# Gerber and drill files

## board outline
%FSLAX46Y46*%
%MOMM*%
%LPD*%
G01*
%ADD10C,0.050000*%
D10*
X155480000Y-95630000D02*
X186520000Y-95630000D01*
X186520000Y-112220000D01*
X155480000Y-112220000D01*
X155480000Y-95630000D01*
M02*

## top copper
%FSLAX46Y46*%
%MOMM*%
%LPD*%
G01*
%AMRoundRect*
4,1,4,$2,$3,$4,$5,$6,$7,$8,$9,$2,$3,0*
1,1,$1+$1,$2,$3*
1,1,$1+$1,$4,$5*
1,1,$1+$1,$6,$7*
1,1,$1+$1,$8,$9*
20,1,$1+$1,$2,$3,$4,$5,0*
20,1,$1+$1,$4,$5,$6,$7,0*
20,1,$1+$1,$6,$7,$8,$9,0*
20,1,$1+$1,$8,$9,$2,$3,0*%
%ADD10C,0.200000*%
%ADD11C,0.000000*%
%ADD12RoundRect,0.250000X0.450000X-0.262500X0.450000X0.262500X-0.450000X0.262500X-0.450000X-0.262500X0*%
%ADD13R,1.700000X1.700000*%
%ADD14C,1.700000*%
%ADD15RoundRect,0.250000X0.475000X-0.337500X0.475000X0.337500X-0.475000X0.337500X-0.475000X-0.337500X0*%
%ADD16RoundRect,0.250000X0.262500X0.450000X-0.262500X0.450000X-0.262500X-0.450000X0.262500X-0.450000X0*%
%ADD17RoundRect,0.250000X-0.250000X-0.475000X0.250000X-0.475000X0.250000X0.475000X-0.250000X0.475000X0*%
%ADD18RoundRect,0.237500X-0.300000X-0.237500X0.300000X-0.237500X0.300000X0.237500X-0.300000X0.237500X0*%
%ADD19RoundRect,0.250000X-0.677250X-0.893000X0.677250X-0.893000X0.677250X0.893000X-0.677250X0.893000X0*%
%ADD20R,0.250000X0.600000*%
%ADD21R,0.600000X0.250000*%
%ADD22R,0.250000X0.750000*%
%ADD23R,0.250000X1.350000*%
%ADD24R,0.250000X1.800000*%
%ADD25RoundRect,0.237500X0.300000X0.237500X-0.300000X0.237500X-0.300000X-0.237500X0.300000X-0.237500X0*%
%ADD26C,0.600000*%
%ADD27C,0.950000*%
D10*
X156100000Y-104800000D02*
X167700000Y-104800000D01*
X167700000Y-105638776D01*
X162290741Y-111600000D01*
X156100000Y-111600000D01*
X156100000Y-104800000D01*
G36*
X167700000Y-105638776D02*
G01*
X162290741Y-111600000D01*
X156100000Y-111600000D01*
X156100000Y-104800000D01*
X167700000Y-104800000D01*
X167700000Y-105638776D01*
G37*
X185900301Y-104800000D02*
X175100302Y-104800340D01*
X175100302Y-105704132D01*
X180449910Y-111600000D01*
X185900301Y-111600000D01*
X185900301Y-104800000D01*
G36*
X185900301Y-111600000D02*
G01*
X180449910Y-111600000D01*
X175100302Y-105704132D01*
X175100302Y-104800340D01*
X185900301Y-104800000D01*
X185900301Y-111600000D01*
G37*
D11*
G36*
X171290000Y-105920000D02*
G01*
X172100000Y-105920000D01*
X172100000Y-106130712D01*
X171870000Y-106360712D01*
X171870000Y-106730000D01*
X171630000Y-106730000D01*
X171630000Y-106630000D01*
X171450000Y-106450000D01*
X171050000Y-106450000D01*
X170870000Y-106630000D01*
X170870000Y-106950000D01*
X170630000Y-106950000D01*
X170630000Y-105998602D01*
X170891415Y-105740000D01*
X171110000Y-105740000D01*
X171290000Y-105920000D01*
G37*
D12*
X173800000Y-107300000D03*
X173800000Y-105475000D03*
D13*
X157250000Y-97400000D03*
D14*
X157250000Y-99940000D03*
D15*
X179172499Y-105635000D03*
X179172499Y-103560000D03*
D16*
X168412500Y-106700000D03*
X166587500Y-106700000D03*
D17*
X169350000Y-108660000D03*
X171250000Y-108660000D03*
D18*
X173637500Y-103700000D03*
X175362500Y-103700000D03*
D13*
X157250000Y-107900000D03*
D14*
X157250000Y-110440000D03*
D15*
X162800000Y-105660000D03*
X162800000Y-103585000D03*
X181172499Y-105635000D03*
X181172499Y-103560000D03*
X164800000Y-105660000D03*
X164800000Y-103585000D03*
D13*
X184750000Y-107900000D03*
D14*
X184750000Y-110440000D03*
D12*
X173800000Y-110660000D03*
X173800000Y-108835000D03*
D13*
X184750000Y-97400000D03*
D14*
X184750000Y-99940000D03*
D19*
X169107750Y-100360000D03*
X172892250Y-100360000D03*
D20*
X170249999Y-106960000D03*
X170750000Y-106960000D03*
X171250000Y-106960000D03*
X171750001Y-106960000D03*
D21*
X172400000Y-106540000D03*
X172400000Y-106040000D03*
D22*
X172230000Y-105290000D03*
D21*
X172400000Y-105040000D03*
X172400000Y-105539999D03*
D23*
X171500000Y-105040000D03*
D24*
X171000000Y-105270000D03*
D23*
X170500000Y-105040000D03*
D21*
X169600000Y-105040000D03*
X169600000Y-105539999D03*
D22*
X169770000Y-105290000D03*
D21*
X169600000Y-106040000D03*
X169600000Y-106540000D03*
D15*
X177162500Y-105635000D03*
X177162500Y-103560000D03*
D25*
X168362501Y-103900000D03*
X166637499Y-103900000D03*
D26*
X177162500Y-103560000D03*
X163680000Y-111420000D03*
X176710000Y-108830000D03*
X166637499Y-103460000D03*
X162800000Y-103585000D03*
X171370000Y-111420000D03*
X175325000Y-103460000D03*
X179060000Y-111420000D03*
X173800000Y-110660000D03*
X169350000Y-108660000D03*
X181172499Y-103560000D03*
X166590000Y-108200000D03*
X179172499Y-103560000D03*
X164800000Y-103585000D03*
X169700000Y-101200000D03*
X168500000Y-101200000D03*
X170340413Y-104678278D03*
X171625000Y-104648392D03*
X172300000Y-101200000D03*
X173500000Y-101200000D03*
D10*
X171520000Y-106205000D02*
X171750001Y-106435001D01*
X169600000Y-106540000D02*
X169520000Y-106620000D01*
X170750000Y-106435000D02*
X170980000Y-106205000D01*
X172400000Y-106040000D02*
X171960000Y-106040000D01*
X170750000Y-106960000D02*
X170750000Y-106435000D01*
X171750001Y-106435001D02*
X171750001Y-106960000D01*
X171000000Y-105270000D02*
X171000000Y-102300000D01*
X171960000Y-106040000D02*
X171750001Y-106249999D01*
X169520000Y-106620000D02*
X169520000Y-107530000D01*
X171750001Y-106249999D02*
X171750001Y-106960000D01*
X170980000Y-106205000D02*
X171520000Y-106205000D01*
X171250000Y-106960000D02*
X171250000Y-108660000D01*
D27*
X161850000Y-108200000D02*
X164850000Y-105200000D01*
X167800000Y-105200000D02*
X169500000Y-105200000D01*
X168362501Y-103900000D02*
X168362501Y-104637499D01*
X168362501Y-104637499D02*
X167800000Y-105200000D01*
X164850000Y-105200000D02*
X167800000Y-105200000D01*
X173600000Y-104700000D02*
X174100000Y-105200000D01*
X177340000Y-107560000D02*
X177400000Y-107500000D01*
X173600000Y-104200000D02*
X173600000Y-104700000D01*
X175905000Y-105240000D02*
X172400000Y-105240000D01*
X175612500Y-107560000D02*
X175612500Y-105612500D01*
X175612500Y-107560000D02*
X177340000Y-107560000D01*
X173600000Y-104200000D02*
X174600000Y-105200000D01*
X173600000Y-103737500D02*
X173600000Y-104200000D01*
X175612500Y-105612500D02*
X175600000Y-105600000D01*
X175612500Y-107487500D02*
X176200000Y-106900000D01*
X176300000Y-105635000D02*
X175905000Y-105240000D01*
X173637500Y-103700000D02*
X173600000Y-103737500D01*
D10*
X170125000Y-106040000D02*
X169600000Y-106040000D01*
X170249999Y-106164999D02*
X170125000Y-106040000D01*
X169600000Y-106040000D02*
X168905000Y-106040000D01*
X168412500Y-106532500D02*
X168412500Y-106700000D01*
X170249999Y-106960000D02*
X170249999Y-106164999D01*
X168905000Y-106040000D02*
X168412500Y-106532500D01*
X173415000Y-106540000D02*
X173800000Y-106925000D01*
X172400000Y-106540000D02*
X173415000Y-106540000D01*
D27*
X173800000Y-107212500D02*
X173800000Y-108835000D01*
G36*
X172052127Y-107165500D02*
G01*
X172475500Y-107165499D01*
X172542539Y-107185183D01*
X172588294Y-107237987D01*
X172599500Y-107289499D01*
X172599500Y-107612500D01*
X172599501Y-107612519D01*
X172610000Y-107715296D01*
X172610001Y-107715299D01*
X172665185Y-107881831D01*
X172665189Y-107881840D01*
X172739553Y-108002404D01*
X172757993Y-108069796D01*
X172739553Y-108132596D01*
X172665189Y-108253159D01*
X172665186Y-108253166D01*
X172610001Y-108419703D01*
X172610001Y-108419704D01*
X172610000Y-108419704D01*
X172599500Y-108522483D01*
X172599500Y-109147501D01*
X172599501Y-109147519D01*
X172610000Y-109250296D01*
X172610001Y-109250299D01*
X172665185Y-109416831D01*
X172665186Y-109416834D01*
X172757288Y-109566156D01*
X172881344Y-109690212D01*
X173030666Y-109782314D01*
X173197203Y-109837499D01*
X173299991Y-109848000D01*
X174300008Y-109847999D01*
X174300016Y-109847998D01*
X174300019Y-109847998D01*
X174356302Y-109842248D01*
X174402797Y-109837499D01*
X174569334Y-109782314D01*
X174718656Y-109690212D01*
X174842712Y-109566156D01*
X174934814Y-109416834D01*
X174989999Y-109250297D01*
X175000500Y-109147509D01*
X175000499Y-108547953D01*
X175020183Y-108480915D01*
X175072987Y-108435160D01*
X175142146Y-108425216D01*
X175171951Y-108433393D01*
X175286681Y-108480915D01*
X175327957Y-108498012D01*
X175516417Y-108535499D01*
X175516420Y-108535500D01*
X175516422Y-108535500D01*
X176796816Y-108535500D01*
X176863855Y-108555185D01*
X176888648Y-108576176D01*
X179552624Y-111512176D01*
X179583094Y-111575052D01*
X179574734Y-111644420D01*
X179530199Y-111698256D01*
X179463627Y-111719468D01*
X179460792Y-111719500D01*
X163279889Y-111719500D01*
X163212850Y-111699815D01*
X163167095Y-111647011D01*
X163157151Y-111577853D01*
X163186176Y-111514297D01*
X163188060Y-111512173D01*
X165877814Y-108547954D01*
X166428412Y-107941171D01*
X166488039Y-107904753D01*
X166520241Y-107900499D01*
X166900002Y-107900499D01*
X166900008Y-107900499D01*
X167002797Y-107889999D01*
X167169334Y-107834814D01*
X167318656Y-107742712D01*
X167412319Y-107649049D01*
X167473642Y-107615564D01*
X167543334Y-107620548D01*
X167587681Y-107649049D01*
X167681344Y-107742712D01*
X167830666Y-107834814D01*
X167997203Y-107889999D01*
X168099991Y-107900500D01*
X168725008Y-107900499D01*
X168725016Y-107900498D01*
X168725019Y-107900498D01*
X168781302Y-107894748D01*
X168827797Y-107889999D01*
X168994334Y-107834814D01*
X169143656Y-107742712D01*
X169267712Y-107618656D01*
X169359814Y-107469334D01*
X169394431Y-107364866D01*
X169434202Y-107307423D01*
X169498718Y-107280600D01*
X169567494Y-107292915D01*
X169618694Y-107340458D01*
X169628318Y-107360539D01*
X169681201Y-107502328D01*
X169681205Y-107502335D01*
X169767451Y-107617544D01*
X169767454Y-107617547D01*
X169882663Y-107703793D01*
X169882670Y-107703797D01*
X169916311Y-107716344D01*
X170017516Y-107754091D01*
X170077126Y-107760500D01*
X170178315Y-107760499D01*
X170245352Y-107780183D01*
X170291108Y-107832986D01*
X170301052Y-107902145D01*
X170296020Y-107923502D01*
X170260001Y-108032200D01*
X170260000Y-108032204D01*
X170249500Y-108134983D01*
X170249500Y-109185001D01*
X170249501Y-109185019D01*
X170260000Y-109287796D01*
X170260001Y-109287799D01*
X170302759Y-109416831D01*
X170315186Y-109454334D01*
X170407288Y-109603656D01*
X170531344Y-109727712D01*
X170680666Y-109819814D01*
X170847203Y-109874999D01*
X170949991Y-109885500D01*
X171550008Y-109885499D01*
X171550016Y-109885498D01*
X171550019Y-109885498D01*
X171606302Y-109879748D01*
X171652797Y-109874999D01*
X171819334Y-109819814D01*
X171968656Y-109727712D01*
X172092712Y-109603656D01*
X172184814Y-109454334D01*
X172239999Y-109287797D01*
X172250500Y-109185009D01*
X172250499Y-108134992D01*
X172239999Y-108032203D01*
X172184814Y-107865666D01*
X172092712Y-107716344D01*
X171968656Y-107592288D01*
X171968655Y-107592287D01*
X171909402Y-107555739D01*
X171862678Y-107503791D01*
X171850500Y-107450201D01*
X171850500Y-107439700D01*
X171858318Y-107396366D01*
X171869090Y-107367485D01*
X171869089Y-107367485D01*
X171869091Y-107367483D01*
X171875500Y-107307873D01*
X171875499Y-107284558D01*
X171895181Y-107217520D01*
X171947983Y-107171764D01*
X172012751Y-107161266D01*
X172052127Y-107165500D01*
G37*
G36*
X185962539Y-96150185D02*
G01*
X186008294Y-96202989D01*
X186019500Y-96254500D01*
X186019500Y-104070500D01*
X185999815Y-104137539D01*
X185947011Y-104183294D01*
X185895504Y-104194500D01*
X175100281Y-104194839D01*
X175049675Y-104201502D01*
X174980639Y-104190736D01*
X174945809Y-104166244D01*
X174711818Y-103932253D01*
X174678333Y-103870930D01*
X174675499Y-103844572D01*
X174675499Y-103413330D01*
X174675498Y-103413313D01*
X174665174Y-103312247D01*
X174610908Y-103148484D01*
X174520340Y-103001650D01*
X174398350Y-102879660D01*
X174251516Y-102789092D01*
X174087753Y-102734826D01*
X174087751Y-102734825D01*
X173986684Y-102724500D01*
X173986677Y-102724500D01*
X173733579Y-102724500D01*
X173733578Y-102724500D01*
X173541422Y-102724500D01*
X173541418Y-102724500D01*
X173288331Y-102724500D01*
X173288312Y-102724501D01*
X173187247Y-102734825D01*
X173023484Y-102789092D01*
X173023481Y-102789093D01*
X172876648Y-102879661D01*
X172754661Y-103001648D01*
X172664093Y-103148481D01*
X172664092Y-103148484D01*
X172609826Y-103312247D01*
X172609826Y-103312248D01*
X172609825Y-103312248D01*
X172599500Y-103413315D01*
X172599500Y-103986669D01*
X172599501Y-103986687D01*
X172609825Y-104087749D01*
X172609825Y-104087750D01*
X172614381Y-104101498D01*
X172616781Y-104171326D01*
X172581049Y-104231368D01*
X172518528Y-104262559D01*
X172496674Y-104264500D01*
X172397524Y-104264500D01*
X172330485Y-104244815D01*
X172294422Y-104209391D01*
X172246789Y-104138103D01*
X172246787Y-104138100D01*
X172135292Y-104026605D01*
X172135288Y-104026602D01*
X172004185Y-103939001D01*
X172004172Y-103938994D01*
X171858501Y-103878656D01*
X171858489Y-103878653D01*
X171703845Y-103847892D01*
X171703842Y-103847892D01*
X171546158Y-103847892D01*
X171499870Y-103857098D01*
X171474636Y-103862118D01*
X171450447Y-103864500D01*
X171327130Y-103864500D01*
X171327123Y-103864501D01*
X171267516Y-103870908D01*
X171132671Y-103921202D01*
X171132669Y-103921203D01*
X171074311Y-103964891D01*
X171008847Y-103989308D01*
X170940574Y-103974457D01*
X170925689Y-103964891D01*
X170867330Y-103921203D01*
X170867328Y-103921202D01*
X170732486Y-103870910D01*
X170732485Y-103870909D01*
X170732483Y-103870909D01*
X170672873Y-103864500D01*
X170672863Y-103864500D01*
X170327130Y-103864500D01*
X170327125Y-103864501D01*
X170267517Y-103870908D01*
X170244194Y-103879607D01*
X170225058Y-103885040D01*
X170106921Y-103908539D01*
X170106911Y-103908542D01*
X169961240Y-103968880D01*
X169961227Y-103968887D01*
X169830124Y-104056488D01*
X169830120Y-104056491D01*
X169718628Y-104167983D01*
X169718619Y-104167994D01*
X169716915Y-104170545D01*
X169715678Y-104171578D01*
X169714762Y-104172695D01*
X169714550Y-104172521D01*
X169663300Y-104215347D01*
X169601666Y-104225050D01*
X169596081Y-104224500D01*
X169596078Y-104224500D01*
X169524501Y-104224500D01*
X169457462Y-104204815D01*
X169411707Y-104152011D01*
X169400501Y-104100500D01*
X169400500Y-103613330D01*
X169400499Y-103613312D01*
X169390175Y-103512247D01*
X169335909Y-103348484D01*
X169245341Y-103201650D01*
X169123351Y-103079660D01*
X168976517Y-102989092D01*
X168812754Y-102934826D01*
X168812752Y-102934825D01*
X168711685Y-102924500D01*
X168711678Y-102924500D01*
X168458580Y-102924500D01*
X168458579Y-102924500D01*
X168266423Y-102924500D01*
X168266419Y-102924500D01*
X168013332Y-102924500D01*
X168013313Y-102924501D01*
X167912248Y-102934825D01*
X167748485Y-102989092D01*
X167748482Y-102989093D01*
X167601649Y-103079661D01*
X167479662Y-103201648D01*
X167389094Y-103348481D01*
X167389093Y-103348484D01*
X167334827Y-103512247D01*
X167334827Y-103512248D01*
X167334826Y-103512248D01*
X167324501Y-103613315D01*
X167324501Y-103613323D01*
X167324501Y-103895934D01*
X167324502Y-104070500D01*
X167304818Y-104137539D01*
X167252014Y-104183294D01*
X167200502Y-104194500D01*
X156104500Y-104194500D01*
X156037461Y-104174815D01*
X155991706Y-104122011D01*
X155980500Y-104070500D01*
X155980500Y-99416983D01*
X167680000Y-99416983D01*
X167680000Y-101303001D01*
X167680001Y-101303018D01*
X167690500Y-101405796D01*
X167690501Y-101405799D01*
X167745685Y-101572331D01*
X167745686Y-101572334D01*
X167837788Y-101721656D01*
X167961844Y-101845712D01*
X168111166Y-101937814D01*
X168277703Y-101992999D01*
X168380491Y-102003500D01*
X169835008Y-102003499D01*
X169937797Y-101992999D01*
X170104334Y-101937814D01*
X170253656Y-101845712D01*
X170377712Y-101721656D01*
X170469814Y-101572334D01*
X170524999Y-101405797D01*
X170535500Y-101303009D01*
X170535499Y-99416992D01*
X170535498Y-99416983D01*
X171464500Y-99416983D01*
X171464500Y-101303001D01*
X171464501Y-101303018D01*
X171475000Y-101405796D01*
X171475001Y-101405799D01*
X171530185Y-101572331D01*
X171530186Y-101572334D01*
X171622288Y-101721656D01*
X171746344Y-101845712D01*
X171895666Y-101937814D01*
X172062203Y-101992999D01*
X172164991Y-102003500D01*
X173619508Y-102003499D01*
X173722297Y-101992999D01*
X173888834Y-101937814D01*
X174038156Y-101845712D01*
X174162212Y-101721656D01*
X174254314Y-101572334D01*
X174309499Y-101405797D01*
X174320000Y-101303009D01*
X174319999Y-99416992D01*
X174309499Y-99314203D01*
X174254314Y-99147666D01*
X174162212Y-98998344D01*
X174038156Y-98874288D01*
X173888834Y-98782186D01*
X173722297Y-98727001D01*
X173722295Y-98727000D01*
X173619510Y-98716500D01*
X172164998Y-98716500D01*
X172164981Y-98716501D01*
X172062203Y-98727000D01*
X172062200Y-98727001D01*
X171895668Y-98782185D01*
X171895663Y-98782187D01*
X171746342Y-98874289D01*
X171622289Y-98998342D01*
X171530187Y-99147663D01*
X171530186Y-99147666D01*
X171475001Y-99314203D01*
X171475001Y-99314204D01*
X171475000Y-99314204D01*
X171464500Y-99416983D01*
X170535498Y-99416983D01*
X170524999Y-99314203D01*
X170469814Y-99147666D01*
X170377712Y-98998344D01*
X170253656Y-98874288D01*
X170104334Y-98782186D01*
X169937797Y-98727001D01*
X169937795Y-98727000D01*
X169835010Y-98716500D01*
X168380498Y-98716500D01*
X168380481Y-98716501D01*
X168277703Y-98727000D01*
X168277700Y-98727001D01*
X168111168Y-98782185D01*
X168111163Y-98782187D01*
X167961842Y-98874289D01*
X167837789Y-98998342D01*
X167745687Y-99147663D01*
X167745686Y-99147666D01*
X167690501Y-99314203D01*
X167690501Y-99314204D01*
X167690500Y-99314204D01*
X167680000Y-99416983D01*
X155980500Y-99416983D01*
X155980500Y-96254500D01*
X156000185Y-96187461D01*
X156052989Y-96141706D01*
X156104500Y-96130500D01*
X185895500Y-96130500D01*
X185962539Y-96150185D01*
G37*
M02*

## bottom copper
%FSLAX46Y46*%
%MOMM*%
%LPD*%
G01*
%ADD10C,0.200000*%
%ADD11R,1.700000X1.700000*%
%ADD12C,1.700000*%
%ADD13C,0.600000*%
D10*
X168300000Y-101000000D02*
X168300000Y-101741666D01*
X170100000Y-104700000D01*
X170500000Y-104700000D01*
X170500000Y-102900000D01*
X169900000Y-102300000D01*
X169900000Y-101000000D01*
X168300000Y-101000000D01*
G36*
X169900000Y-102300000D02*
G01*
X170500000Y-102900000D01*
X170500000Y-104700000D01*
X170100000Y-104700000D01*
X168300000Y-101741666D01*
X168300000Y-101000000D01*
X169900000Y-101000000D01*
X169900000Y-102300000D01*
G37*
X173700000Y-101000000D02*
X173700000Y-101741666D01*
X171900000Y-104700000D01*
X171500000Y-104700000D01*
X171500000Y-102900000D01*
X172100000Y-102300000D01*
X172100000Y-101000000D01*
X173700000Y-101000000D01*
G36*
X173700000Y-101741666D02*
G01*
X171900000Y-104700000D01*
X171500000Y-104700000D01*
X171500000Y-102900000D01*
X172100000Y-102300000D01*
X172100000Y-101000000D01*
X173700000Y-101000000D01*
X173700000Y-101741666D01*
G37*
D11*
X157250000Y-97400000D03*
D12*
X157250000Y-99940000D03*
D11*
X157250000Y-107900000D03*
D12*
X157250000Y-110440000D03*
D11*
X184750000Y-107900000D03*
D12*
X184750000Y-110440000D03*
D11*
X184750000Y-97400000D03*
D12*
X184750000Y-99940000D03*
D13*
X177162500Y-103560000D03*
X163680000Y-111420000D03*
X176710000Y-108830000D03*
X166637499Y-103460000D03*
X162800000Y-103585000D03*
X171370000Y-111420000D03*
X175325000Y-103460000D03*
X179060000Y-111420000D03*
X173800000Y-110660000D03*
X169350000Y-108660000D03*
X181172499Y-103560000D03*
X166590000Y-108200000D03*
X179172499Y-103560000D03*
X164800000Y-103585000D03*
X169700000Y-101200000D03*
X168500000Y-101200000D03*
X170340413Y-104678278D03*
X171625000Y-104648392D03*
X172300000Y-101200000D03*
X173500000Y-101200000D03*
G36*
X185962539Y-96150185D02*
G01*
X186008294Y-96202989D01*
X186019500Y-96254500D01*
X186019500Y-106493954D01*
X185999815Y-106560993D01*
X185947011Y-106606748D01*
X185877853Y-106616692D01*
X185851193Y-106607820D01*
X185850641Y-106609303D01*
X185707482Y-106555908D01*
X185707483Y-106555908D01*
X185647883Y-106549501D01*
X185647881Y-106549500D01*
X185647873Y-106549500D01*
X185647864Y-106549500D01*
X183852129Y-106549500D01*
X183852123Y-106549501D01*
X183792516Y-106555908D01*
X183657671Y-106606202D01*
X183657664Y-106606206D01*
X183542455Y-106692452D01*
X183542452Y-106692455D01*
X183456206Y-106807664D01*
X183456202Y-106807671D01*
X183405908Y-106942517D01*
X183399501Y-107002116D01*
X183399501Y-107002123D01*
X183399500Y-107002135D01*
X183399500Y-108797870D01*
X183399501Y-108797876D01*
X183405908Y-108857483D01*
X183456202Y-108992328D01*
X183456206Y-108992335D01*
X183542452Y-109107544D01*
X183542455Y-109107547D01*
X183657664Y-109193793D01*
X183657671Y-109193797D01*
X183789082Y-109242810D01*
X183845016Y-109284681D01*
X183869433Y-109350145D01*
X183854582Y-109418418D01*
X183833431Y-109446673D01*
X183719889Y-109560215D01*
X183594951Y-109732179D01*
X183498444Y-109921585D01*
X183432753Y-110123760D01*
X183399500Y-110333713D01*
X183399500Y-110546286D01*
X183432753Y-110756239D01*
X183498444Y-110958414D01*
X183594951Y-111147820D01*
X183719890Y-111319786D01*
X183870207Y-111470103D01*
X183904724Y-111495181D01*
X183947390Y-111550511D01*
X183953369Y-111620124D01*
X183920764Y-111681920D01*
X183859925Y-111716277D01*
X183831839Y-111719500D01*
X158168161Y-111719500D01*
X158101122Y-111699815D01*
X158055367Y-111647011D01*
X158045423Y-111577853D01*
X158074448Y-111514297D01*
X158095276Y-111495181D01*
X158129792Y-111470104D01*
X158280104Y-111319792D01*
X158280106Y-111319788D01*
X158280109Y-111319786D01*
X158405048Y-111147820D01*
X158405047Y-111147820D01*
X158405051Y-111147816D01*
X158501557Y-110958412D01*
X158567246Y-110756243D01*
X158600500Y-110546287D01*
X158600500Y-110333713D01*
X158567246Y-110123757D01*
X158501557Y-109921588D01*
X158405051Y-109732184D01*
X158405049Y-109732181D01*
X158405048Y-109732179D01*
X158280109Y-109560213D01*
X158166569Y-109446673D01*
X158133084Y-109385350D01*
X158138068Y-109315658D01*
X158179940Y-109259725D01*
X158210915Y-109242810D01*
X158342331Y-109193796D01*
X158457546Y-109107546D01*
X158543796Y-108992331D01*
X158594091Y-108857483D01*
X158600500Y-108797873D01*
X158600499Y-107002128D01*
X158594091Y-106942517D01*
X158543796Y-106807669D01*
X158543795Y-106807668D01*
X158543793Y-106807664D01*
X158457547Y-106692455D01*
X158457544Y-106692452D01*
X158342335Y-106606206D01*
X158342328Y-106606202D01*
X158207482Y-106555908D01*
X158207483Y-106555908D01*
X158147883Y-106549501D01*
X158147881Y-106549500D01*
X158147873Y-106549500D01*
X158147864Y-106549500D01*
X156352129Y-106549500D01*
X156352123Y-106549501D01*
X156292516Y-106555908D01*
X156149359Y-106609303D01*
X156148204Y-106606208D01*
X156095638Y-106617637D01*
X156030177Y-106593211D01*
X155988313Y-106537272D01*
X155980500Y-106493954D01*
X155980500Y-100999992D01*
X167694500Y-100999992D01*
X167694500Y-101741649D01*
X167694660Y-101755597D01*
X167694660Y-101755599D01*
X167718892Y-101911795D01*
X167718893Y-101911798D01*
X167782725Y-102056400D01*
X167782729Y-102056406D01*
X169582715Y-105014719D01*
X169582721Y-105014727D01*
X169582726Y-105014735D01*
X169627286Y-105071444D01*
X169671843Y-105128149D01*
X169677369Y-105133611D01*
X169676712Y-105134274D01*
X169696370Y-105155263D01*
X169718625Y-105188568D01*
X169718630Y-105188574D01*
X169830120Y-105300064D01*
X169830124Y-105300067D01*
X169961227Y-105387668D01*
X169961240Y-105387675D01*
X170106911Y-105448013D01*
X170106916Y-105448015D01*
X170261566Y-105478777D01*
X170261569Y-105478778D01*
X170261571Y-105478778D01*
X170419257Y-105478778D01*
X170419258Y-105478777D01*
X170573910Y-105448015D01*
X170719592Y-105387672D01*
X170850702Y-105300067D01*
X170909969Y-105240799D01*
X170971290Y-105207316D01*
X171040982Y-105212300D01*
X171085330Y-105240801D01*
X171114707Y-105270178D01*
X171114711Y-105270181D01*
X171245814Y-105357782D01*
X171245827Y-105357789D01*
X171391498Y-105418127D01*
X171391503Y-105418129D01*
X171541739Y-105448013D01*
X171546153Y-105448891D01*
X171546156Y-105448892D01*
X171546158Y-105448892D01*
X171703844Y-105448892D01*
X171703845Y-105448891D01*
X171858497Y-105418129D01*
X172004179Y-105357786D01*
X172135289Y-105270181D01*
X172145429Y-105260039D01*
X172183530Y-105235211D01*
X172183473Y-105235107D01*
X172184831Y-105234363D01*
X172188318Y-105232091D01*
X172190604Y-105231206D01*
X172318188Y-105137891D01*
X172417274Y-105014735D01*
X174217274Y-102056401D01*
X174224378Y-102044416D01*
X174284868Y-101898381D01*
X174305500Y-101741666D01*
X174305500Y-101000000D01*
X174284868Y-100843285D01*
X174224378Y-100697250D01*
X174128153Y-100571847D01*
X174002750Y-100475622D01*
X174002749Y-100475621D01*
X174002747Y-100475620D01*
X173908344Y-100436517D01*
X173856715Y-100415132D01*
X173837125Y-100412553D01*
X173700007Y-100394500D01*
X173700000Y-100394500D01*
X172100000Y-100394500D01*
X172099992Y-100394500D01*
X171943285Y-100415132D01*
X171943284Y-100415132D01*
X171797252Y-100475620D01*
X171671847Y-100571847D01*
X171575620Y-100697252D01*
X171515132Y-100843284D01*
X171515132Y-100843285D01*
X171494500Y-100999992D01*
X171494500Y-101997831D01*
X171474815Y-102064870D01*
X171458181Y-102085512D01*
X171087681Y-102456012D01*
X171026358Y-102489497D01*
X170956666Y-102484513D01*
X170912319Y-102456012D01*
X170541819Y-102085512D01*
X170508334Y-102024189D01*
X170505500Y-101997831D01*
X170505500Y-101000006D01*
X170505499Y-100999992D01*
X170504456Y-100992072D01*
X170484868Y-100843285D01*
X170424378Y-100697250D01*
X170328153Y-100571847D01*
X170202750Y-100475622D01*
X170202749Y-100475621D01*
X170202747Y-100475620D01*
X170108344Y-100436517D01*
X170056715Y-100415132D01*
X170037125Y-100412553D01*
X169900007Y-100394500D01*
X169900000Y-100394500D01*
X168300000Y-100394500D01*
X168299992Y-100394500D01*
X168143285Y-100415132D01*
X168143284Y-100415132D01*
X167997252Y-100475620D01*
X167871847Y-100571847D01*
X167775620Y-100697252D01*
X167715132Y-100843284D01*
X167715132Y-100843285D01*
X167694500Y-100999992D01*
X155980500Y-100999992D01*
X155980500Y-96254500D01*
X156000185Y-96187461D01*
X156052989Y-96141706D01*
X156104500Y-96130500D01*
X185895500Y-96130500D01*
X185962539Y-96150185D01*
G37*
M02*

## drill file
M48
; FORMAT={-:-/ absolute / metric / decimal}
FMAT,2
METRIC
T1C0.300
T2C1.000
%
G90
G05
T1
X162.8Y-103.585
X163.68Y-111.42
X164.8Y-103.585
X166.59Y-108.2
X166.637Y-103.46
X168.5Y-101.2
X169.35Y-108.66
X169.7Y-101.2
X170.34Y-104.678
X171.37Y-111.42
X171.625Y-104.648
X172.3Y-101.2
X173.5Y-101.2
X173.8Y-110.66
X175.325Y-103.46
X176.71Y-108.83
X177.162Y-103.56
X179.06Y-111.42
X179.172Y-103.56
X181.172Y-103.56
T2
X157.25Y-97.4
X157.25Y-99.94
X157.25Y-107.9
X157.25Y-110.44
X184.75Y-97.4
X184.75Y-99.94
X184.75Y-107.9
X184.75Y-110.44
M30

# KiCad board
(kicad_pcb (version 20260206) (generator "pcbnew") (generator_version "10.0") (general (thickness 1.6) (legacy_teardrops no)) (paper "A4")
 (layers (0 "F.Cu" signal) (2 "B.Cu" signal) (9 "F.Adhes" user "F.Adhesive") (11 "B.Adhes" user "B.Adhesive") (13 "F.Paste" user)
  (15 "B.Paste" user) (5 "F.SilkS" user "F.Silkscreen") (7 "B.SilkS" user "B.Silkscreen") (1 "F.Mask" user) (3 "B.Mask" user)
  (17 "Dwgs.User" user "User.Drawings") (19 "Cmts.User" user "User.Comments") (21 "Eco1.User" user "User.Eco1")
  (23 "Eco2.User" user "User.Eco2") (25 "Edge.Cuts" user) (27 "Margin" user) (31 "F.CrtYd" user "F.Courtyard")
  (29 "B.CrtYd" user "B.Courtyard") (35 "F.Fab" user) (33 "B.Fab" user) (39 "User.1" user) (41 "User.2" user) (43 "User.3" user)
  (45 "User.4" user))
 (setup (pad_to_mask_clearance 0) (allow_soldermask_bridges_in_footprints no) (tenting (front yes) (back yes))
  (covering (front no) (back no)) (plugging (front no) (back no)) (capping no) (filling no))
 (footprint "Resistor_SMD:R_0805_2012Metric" (layer "F.Cu") (at 173.8 106.3875 90)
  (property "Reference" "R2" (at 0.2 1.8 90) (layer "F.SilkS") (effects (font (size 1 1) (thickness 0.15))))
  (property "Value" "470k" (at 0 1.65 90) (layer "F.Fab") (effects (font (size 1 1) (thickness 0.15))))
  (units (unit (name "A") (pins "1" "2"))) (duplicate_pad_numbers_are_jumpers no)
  (pad "1" smd roundrect (at -0.9125 0 90) (size 1.025 1.4) (layers "F.Cu" "F.Mask" "F.Paste") (roundrect_rratio 0.243902)
   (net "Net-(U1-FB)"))
  (pad "2" smd roundrect (at 0.9125 0 90) (size 1.025 1.4) (layers "F.Cu" "F.Mask" "F.Paste") (roundrect_rratio 0.243902) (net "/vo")))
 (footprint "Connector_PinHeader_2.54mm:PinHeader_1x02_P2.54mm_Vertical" (layer "F.Cu") (at 157.25 97.4)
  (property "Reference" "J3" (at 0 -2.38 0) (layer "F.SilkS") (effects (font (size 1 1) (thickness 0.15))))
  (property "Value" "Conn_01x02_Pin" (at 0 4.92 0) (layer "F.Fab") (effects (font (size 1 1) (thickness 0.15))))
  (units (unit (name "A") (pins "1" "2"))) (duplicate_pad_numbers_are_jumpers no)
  (pad "1" thru_hole rect (at 0 0) (size 1.7 1.7) (drill 1) (layers "*.Cu" "*.Mask") (remove_unused_layers no) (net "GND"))
  (pad "2" thru_hole circle (at 0 2.54) (size 1.7 1.7) (drill 1) (layers "*.Cu" "*.Mask") (remove_unused_layers no) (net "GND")))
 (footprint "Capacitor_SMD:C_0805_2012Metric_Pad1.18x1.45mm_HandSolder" (layer "F.Cu") (at 179.172499 104.5975 90)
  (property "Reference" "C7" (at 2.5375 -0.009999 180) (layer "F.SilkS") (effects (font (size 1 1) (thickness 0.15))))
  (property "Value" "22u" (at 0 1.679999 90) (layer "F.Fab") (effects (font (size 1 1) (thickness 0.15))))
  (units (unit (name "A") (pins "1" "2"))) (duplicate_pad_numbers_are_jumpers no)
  (pad "1" smd roundrect (at -1.0375 0 90) (size 1.175 1.45) (layers "F.Cu" "F.Mask" "F.Paste") (roundrect_rratio 0.212766) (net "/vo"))
  (pad "2" smd roundrect (at 1.0375 0 90) (size 1.175 1.45) (layers "F.Cu" "F.Mask" "F.Paste") (roundrect_rratio 0.212766) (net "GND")))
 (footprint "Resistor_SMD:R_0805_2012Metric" (layer "F.Cu") (at 167.5 106.7 180)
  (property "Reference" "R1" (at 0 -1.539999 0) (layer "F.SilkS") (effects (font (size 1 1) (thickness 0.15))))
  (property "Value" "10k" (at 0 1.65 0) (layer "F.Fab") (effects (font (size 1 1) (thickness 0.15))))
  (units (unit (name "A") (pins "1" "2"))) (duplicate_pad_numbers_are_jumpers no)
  (pad "1" smd roundrect (at -0.9125 0 180) (size 1.025 1.4) (layers "F.Cu" "F.Mask" "F.Paste") (roundrect_rratio 0.243902)
   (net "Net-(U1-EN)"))
  (pad "2" smd roundrect (at 0.9125 0 180) (size 1.025 1.4) (layers "F.Cu" "F.Mask" "F.Paste") (roundrect_rratio 0.243902) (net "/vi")))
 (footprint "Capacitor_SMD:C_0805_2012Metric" (layer "F.Cu") (at 170.3 108.66)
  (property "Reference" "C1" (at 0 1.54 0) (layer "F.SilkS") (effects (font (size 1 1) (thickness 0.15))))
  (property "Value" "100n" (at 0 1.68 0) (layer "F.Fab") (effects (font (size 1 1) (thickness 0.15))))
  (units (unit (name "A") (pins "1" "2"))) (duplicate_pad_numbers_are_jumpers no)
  (pad "1" smd roundrect (at -0.95 0) (size 1 1.45) (layers "F.Cu" "F.Mask" "F.Paste") (roundrect_rratio 0.25) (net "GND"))
  (pad "2" smd roundrect (at 0.95 0) (size 1 1.45) (layers "F.Cu" "F.Mask" "F.Paste") (roundrect_rratio 0.25) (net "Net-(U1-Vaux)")))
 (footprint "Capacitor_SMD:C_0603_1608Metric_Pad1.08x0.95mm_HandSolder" (layer "F.Cu") (at 174.5 103.7)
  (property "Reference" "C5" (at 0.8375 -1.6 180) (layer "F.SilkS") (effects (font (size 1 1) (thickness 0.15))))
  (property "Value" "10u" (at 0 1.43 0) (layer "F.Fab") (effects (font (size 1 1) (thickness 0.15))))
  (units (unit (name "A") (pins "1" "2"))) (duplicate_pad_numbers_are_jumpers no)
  (pad "1" smd roundrect (at -0.8625 0) (size 1.075 0.95) (layers "F.Cu" "F.Mask" "F.Paste") (roundrect_rratio 0.25) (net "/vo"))
  (pad "2" smd roundrect (at 0.8625 0) (size 1.075 0.95) (layers "F.Cu" "F.Mask" "F.Paste") (roundrect_rratio 0.25) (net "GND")))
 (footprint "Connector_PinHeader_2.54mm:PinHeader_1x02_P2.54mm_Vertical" (layer "F.Cu") (at 157.25 107.9)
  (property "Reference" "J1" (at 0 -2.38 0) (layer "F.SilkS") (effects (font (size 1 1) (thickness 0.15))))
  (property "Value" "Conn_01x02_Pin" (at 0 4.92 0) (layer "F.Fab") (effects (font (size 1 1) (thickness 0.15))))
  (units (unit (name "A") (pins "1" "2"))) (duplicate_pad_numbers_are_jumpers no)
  (pad "1" thru_hole rect (at 0 0) (size 1.7 1.7) (drill 1) (layers "*.Cu" "*.Mask") (remove_unused_layers no) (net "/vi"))
  (pad "2" thru_hole circle (at 0 2.54) (size 1.7 1.7) (drill 1) (layers "*.Cu" "*.Mask") (remove_unused_layers no) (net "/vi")))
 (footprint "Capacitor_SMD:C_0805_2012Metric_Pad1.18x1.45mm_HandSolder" (layer "F.Cu") (at 162.8 104.6225 90)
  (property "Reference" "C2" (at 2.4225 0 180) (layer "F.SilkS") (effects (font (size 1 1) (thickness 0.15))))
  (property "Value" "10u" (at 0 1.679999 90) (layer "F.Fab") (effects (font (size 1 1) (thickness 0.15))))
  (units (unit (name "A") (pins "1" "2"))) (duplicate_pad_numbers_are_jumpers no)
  (pad "1" smd roundrect (at -1.0375 0 90) (size 1.175 1.45) (layers "F.Cu" "F.Mask" "F.Paste") (roundrect_rratio 0.212766) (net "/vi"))
  (pad "2" smd roundrect (at 1.0375 0 90) (size 1.175 1.45) (layers "F.Cu" "F.Mask" "F.Paste") (roundrect_rratio 0.212766) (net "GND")))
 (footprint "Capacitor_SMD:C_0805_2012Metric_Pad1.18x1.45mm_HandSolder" (layer "F.Cu") (at 181.172499 104.5975 90)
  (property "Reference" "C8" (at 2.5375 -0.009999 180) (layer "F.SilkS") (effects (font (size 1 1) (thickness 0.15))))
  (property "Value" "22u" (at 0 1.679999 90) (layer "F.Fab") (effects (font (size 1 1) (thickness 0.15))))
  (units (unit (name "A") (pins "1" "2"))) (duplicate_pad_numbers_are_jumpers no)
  (pad "1" smd roundrect (at -1.0375 0 90) (size 1.175 1.45) (layers "F.Cu" "F.Mask" "F.Paste") (roundrect_rratio 0.212766) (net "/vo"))
  (pad "2" smd roundrect (at 1.0375 0 90) (size 1.175 1.45) (layers "F.Cu" "F.Mask" "F.Paste") (roundrect_rratio 0.212766) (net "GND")))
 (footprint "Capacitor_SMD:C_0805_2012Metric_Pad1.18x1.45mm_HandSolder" (layer "F.Cu") (at 164.8 104.6225 90)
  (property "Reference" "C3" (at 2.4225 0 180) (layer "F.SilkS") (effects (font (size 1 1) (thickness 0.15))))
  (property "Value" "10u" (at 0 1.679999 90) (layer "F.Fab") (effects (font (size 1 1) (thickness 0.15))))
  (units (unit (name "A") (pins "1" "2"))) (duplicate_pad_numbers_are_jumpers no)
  (pad "1" smd roundrect (at -1.0375 0 90) (size 1.175 1.45) (layers "F.Cu" "F.Mask" "F.Paste") (roundrect_rratio 0.212766) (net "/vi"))
  (pad "2" smd roundrect (at 1.0375 0 90) (size 1.175 1.45) (layers "F.Cu" "F.Mask" "F.Paste") (roundrect_rratio 0.212766) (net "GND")))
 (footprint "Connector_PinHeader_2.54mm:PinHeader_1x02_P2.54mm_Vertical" (layer "F.Cu") (at 184.75 107.9)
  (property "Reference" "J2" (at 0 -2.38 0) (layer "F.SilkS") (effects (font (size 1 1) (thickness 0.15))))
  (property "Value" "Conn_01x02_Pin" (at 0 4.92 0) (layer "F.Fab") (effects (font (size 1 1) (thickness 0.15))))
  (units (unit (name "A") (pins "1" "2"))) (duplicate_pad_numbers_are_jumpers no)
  (pad "1" thru_hole rect (at 0 0) (size 1.7 1.7) (drill 1) (layers "*.Cu" "*.Mask") (remove_unused_layers no) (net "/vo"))
  (pad "2" thru_hole circle (at 0 2.54) (size 1.7 1.7) (drill 1) (layers "*.Cu" "*.Mask") (remove_unused_layers no) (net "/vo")))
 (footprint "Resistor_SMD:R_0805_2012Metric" (layer "F.Cu") (at 173.8 109.7475 90)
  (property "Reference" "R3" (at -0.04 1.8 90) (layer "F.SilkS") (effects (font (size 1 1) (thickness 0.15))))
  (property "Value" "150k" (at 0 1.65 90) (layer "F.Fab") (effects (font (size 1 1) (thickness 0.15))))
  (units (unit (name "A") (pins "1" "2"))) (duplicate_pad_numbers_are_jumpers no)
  (pad "1" smd roundrect (at -0.9125 0 90) (size 1.025 1.4) (layers "F.Cu" "F.Mask" "F.Paste") (roundrect_rratio 0.243902) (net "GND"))
  (pad "2" smd roundrect (at 0.9125 0 90) (size 1.025 1.4) (layers "F.Cu" "F.Mask" "F.Paste") (roundrect_rratio 0.243902)
   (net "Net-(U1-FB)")))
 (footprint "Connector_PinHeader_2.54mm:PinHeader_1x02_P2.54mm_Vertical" (layer "F.Cu") (at 184.75 97.4)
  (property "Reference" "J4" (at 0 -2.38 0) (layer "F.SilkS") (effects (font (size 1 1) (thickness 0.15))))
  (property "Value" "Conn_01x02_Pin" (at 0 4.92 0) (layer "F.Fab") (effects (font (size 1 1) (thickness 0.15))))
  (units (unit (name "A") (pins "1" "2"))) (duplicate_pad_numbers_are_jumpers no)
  (pad "1" thru_hole rect (at 0 0) (size 1.7 1.7) (drill 1) (layers "*.Cu" "*.Mask") (remove_unused_layers no) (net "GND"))
  (pad "2" thru_hole circle (at 0 2.54) (size 1.7 1.7) (drill 1) (layers "*.Cu" "*.Mask") (remove_unused_layers no) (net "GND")))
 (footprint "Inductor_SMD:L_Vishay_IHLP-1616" (layer "F.Cu") (at 171 100.36)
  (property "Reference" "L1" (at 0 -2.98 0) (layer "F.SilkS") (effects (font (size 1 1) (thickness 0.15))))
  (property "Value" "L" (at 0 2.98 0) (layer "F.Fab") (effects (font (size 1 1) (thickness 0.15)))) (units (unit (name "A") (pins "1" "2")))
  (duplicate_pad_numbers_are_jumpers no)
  (pad "1" smd roundrect (at -1.89225 0) (size 1.8545 2.286) (layers "F.Cu" "F.Mask" "F.Paste") (roundrect_rratio 0.134807)
   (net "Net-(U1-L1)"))
  (pad "2" smd roundrect (at 1.89225 0) (size 1.8545 2.286) (layers "F.Cu" "F.Mask" "F.Paste") (roundrect_rratio 0.134807)
   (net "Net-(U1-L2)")))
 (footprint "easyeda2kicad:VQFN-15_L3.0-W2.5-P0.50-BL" (layer "F.Cu") (at 171 106)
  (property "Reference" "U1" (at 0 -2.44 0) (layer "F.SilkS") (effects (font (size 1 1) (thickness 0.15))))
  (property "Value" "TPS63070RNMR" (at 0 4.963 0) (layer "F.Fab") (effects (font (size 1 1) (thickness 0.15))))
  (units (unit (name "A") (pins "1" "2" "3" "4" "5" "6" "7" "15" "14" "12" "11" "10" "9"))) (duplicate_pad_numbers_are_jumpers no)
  (pad "1" smd rect (at -0.750001 0.96 180) (size 0.25 0.6) (layers "F.Cu" "F.Mask" "F.Paste") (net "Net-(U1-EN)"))
  (pad "2" smd rect (at -0.25 0.96 180) (size 0.25 0.6) (layers "F.Cu" "F.Mask" "F.Paste") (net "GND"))
  (pad "3" smd rect (at 0.25 0.96 180) (size 0.25 0.6) (layers "F.Cu" "F.Mask" "F.Paste") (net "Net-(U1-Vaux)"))
  (pad "4" smd rect (at 0.750001 0.96 180) (size 0.25 0.6) (layers "F.Cu" "F.Mask" "F.Paste") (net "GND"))
  (pad "5" smd rect (at 1.4 0.54 270) (size 0.25 0.6) (layers "F.Cu" "F.Mask" "F.Paste") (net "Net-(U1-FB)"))
  (pad "6" smd rect (at 1.4 0.04 270) (size 0.25 0.6) (layers "F.Cu" "F.Mask" "F.Paste") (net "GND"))
  (pad "7" smd rect (at 1.23 -0.71) (size 0.25 0.75) (layers "F.Cu" "F.Mask" "F.Paste") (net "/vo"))
  (pad "7" smd rect (at 1.4 -0.96 270) (size 0.25 0.6) (layers "F.Cu" "F.Mask" "F.Paste") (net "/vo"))
  (pad "7" smd rect (at 1.4 -0.460001 270) (size 0.25 0.6) (layers "F.Cu" "F.Mask" "F.Paste") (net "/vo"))
  (pad "9" smd rect (at 0.5 -0.96) (size 0.25 1.35) (layers "F.Cu" "F.Mask" "F.Paste") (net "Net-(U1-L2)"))
  (pad "10" smd rect (at 0 -0.73) (size 0.25 1.8) (layers "F.Cu" "F.Mask" "F.Paste") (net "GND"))
  (pad "11" smd rect (at -0.5 -0.96) (size 0.25 1.35) (layers "F.Cu" "F.Mask" "F.Paste") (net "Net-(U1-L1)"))
  (pad "12" smd rect (at -1.4 -0.96 90) (size 0.25 0.6) (layers "F.Cu" "F.Mask" "F.Paste") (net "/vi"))
  (pad "12" smd rect (at -1.4 -0.460001 90) (size 0.25 0.6) (layers "F.Cu" "F.Mask" "F.Paste") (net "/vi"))
  (pad "12" smd rect (at -1.23 -0.71 180) (size 0.25 0.75) (layers "F.Cu" "F.Mask" "F.Paste") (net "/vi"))
  (pad "14" smd rect (at -1.4 0.04 90) (size 0.25 0.6) (layers "F.Cu" "F.Mask" "F.Paste") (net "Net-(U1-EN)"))
  (pad "15" smd rect (at -1.4 0.54 90) (size 0.25 0.6) (layers "F.Cu" "F.Mask" "F.Paste") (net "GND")))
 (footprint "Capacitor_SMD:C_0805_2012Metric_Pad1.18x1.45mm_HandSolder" (layer "F.Cu") (at 177.1625 104.5975 90)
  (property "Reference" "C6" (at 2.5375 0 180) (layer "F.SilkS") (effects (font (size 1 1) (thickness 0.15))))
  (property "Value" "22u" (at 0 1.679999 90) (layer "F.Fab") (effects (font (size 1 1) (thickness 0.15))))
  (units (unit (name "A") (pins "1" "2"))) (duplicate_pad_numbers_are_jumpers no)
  (pad "1" smd roundrect (at -1.0375 0 90) (size 1.175 1.45) (layers "F.Cu" "F.Mask" "F.Paste") (roundrect_rratio 0.212766) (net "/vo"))
  (pad "2" smd roundrect (at 1.0375 0 90) (size 1.175 1.45) (layers "F.Cu" "F.Mask" "F.Paste") (roundrect_rratio 0.212766) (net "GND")))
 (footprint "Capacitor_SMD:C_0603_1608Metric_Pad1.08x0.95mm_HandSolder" (layer "F.Cu") (at 167.5 103.9 180)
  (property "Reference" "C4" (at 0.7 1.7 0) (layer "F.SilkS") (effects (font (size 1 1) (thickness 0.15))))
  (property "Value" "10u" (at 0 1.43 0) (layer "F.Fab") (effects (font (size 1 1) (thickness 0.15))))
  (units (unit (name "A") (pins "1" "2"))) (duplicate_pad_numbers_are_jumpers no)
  (pad "1" smd roundrect (at -0.862501 0 180) (size 1.075 0.95) (layers "F.Cu" "F.Mask" "F.Paste") (roundrect_rratio 0.25) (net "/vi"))
  (pad "2" smd roundrect (at 0.862501 0 180) (size 1.075 0.95) (layers "F.Cu" "F.Mask" "F.Paste") (roundrect_rratio 0.25) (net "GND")))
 (gr_poly
  (pts (xy 156.1 104.8) (xy 167.7 104.8) (xy 167.7 105.638776) (xy 162.290741 111.6) (xy 156.1 111.6)) (stroke (width 0.2) (type solid))
  (fill yes) (layer "F.Cu") (net "/vi"))
 (gr_poly
  (pts (xy 185.900301 104.8) (xy 175.100302 104.80034) (xy 175.100302 105.704132) (xy 180.44991 111.6) (xy 185.900301 111.6))
  (stroke (width 0.2) (type solid)) (fill yes) (layer "F.Cu") (net "/vo"))
 (gr_poly
  (pts (xy 172.1 105.92) (xy 171.29 105.92) (xy 171.11 105.74) (xy 170.891415 105.74) (xy 170.63 105.998602) (xy 170.63 106.95)
   (xy 170.87 106.95) (xy 170.87 106.63) (xy 171.05 106.45) (xy 171.45 106.45) (xy 171.63 106.63) (xy 171.63 106.73) (xy 171.87 106.73)
   (xy 171.87 106.360712) (xy 172.1 106.130712))
  (stroke (width 0) (type solid)) (fill yes) (layer "F.Cu") (net "GND"))
 (gr_poly
  (pts (xy 168.3 101) (xy 168.3 101.741666) (xy 170.1 104.7) (xy 170.5 104.7) (xy 170.5 102.9) (xy 169.9 102.3) (xy 169.9 101))
  (stroke (width 0.2) (type solid)) (fill yes) (layer "B.Cu") (net "Net-(U1-L1)"))
 (gr_poly
  (pts (xy 173.7 101) (xy 173.7 101.741666) (xy 171.9 104.7) (xy 171.5 104.7) (xy 171.5 102.9) (xy 172.1 102.3) (xy 172.1 101))
  (stroke (width 0.2) (type solid)) (fill yes) (layer "B.Cu") (net "Net-(U1-L2)"))
 (gr_rect (start 155.48 95.63) (end 186.52 112.22) (stroke (width 0.05) (type default)) (fill no) (layer "Edge.Cuts"))
 (segment (start 171.52 106.205) (end 171.750001 106.435001) (width 0.2) (layer "F.Cu") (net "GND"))
 (segment (start 169.6 106.54) (end 169.52 106.62) (width 0.2) (layer "F.Cu") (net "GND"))
 (segment (start 170.75 106.435) (end 170.98 106.205) (width 0.2) (layer "F.Cu") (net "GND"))
 (segment (start 172.4 106.04) (end 171.96 106.04) (width 0.2) (layer "F.Cu") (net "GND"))
 (segment (start 170.75 106.96) (end 170.75 106.435) (width 0.2) (layer "F.Cu") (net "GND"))
 (segment (start 171.750001 106.435001) (end 171.750001 106.96) (width 0.2) (layer "F.Cu") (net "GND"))
 (segment (start 171 105.27) (end 171 102.3) (width 0.2) (layer "F.Cu") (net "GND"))
 (segment (start 171.96 106.04) (end 171.750001 106.249999) (width 0.2) (layer "F.Cu") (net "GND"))
 (segment (start 169.52 106.62) (end 169.52 107.53) (width 0.2) (layer "F.Cu") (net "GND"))
 (segment (start 171.750001 106.249999) (end 171.750001 106.96) (width 0.2) (layer "F.Cu") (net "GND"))
 (segment (start 170.98 106.205) (end 171.52 106.205) (width 0.2) (layer "F.Cu") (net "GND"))
 (via (at 177.1625 103.56) (size 0.6) (drill 0.3) (layers "F.Cu" "B.Cu") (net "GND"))
 (via (at 163.68 111.42) (size 0.6) (drill 0.3) (layers "F.Cu" "B.Cu") (free yes) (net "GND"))
 (via (at 176.71 108.83) (size 0.6) (drill 0.3) (layers "F.Cu" "B.Cu") (free yes) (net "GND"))
 (via (at 166.637499 103.46) (size 0.6) (drill 0.3) (layers "F.Cu" "B.Cu") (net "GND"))
 (via (at 162.8 103.585) (size 0.6) (drill 0.3) (layers "F.Cu" "B.Cu") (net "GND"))
 (via (at 171.37 111.42) (size 0.6) (drill 0.3) (layers "F.Cu" "B.Cu") (free yes) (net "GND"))
 (via (at 175.325 103.46) (size 0.6) (drill 0.3) (layers "F.Cu" "B.Cu") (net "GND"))
 (via (at 179.06 111.42) (size 0.6) (drill 0.3) (layers "F.Cu" "B.Cu") (free yes) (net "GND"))
 (via (at 173.8 110.66) (size 0.6) (drill 0.3) (layers "F.Cu" "B.Cu") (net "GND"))
 (via (at 169.35 108.66) (size 0.6) (drill 0.3) (layers "F.Cu" "B.Cu") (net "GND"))
 (via (at 181.172499 103.56) (size 0.6) (drill 0.3) (layers "F.Cu" "B.Cu") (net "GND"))
 (via (at 166.59 108.2) (size 0.6) (drill 0.3) (layers "F.Cu" "B.Cu") (free yes) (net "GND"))
 (via (at 179.172499 103.56) (size 0.6) (drill 0.3) (layers "F.Cu" "B.Cu") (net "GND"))
 (via (at 164.8 103.585) (size 0.6) (drill 0.3) (layers "F.Cu" "B.Cu") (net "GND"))
 (segment (start 171.25 106.96) (end 171.25 108.66) (width 0.2) (layer "F.Cu") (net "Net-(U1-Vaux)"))
 (segment (start 161.85 108.2) (end 164.85 105.2) (width 0.95) (layer "F.Cu") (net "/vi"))
 (segment (start 167.8 105.2) (end 169.5 105.2) (width 0.95) (layer "F.Cu") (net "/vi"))
 (segment (start 168.362501 103.9) (end 168.362501 104.637499) (width 0.95) (layer "F.Cu") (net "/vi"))
 (segment (start 168.362501 104.637499) (end 167.8 105.2) (width 0.95) (layer "F.Cu") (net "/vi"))
 (segment (start 164.85 105.2) (end 167.8 105.2) (width 0.95) (layer "F.Cu") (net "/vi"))
 (segment (start 173.6 104.7) (end 174.1 105.2) (width 0.95) (layer "F.Cu") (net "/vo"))
 (segment (start 177.34 107.56) (end 177.4 107.5) (width 0.95) (layer "F.Cu") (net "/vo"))
 (segment (start 173.6 104.2) (end 173.6 104.7) (width 0.95) (layer "F.Cu") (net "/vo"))
 (segment (start 175.905 105.24) (end 172.4 105.24) (width 0.95) (layer "F.Cu") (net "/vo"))
 (segment (start 175.6125 107.56) (end 175.6125 105.6125) (width 0.95) (layer "F.Cu") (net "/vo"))
 (segment (start 175.6125 107.56) (end 177.34 107.56) (width 0.95) (layer "F.Cu") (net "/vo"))
 (segment (start 173.6 104.2) (end 174.6 105.2) (width 0.95) (layer "F.Cu") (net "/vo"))
 (segment (start 173.6 103.7375) (end 173.6 104.2) (width 0.95) (layer "F.Cu") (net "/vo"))
 (segment (start 175.6125 105.6125) (end 175.6 105.6) (width 0.95) (layer "F.Cu") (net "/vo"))
 (segment (start 175.6125 107.4875) (end 176.2 106.9) (width 0.95) (layer "F.Cu") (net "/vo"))
 (segment (start 176.3 105.635) (end 175.905 105.24) (width 0.95) (layer "F.Cu") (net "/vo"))
 (segment (start 173.6375 103.7) (end 173.6 103.7375) (width 0.95) (layer "F.Cu") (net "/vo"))
 (via (at 169.7 101.2) (size 0.6) (drill 0.3) (layers "F.Cu" "B.Cu") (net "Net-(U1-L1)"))
 (via (at 168.5 101.2) (size 0.6) (drill 0.3) (layers "F.Cu" "B.Cu") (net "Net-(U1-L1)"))
 (via (at 170.340413 104.678278) (size 0.6) (drill 0.3) (layers "F.Cu" "B.Cu") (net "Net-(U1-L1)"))
 (via (at 171.625 104.648392) (size 0.6) (drill 0.3) (layers "F.Cu" "B.Cu") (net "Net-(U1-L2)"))
 (via (at 172.3 101.2) (size 0.6) (drill 0.3) (layers "F.Cu" "B.Cu") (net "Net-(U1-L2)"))
 (via (at 173.5 101.2) (size 0.6) (drill 0.3) (layers "F.Cu" "B.Cu") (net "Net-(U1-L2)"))
 (segment (start 170.125 106.04) (end 169.6 106.04) (width 0.2) (layer "F.Cu") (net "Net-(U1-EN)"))
 (segment (start 170.249999 106.164999) (end 170.125 106.04) (width 0.2) (layer "F.Cu") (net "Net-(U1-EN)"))
 (segment (start 169.6 106.04) (end 168.905 106.04) (width 0.2) (layer "F.Cu") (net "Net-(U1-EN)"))
 (segment (start 168.4125 106.5325) (end 168.4125 106.7) (width 0.2) (layer "F.Cu") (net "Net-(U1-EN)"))
 (segment (start 170.249999 106.96) (end 170.249999 106.164999) (width 0.2) (layer "F.Cu") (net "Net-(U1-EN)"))
 (segment (start 168.905 106.04) (end 168.4125 106.5325) (width 0.2) (layer "F.Cu") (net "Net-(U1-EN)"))
 (segment (start 173.415 106.54) (end 173.8 106.925) (width 0.2) (layer "F.Cu") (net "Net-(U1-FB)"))
 (segment (start 172.4 106.54) (end 173.415 106.54) (width 0.2) (layer "F.Cu") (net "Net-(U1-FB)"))
 (segment (start 173.8 107.2125) (end 173.8 108.835) (width 0.95) (layer "F.Cu") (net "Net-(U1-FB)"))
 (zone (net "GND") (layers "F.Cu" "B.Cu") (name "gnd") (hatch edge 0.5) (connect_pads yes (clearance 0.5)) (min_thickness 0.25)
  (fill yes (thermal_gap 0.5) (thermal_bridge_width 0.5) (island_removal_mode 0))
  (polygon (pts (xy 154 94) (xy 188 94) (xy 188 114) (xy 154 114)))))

